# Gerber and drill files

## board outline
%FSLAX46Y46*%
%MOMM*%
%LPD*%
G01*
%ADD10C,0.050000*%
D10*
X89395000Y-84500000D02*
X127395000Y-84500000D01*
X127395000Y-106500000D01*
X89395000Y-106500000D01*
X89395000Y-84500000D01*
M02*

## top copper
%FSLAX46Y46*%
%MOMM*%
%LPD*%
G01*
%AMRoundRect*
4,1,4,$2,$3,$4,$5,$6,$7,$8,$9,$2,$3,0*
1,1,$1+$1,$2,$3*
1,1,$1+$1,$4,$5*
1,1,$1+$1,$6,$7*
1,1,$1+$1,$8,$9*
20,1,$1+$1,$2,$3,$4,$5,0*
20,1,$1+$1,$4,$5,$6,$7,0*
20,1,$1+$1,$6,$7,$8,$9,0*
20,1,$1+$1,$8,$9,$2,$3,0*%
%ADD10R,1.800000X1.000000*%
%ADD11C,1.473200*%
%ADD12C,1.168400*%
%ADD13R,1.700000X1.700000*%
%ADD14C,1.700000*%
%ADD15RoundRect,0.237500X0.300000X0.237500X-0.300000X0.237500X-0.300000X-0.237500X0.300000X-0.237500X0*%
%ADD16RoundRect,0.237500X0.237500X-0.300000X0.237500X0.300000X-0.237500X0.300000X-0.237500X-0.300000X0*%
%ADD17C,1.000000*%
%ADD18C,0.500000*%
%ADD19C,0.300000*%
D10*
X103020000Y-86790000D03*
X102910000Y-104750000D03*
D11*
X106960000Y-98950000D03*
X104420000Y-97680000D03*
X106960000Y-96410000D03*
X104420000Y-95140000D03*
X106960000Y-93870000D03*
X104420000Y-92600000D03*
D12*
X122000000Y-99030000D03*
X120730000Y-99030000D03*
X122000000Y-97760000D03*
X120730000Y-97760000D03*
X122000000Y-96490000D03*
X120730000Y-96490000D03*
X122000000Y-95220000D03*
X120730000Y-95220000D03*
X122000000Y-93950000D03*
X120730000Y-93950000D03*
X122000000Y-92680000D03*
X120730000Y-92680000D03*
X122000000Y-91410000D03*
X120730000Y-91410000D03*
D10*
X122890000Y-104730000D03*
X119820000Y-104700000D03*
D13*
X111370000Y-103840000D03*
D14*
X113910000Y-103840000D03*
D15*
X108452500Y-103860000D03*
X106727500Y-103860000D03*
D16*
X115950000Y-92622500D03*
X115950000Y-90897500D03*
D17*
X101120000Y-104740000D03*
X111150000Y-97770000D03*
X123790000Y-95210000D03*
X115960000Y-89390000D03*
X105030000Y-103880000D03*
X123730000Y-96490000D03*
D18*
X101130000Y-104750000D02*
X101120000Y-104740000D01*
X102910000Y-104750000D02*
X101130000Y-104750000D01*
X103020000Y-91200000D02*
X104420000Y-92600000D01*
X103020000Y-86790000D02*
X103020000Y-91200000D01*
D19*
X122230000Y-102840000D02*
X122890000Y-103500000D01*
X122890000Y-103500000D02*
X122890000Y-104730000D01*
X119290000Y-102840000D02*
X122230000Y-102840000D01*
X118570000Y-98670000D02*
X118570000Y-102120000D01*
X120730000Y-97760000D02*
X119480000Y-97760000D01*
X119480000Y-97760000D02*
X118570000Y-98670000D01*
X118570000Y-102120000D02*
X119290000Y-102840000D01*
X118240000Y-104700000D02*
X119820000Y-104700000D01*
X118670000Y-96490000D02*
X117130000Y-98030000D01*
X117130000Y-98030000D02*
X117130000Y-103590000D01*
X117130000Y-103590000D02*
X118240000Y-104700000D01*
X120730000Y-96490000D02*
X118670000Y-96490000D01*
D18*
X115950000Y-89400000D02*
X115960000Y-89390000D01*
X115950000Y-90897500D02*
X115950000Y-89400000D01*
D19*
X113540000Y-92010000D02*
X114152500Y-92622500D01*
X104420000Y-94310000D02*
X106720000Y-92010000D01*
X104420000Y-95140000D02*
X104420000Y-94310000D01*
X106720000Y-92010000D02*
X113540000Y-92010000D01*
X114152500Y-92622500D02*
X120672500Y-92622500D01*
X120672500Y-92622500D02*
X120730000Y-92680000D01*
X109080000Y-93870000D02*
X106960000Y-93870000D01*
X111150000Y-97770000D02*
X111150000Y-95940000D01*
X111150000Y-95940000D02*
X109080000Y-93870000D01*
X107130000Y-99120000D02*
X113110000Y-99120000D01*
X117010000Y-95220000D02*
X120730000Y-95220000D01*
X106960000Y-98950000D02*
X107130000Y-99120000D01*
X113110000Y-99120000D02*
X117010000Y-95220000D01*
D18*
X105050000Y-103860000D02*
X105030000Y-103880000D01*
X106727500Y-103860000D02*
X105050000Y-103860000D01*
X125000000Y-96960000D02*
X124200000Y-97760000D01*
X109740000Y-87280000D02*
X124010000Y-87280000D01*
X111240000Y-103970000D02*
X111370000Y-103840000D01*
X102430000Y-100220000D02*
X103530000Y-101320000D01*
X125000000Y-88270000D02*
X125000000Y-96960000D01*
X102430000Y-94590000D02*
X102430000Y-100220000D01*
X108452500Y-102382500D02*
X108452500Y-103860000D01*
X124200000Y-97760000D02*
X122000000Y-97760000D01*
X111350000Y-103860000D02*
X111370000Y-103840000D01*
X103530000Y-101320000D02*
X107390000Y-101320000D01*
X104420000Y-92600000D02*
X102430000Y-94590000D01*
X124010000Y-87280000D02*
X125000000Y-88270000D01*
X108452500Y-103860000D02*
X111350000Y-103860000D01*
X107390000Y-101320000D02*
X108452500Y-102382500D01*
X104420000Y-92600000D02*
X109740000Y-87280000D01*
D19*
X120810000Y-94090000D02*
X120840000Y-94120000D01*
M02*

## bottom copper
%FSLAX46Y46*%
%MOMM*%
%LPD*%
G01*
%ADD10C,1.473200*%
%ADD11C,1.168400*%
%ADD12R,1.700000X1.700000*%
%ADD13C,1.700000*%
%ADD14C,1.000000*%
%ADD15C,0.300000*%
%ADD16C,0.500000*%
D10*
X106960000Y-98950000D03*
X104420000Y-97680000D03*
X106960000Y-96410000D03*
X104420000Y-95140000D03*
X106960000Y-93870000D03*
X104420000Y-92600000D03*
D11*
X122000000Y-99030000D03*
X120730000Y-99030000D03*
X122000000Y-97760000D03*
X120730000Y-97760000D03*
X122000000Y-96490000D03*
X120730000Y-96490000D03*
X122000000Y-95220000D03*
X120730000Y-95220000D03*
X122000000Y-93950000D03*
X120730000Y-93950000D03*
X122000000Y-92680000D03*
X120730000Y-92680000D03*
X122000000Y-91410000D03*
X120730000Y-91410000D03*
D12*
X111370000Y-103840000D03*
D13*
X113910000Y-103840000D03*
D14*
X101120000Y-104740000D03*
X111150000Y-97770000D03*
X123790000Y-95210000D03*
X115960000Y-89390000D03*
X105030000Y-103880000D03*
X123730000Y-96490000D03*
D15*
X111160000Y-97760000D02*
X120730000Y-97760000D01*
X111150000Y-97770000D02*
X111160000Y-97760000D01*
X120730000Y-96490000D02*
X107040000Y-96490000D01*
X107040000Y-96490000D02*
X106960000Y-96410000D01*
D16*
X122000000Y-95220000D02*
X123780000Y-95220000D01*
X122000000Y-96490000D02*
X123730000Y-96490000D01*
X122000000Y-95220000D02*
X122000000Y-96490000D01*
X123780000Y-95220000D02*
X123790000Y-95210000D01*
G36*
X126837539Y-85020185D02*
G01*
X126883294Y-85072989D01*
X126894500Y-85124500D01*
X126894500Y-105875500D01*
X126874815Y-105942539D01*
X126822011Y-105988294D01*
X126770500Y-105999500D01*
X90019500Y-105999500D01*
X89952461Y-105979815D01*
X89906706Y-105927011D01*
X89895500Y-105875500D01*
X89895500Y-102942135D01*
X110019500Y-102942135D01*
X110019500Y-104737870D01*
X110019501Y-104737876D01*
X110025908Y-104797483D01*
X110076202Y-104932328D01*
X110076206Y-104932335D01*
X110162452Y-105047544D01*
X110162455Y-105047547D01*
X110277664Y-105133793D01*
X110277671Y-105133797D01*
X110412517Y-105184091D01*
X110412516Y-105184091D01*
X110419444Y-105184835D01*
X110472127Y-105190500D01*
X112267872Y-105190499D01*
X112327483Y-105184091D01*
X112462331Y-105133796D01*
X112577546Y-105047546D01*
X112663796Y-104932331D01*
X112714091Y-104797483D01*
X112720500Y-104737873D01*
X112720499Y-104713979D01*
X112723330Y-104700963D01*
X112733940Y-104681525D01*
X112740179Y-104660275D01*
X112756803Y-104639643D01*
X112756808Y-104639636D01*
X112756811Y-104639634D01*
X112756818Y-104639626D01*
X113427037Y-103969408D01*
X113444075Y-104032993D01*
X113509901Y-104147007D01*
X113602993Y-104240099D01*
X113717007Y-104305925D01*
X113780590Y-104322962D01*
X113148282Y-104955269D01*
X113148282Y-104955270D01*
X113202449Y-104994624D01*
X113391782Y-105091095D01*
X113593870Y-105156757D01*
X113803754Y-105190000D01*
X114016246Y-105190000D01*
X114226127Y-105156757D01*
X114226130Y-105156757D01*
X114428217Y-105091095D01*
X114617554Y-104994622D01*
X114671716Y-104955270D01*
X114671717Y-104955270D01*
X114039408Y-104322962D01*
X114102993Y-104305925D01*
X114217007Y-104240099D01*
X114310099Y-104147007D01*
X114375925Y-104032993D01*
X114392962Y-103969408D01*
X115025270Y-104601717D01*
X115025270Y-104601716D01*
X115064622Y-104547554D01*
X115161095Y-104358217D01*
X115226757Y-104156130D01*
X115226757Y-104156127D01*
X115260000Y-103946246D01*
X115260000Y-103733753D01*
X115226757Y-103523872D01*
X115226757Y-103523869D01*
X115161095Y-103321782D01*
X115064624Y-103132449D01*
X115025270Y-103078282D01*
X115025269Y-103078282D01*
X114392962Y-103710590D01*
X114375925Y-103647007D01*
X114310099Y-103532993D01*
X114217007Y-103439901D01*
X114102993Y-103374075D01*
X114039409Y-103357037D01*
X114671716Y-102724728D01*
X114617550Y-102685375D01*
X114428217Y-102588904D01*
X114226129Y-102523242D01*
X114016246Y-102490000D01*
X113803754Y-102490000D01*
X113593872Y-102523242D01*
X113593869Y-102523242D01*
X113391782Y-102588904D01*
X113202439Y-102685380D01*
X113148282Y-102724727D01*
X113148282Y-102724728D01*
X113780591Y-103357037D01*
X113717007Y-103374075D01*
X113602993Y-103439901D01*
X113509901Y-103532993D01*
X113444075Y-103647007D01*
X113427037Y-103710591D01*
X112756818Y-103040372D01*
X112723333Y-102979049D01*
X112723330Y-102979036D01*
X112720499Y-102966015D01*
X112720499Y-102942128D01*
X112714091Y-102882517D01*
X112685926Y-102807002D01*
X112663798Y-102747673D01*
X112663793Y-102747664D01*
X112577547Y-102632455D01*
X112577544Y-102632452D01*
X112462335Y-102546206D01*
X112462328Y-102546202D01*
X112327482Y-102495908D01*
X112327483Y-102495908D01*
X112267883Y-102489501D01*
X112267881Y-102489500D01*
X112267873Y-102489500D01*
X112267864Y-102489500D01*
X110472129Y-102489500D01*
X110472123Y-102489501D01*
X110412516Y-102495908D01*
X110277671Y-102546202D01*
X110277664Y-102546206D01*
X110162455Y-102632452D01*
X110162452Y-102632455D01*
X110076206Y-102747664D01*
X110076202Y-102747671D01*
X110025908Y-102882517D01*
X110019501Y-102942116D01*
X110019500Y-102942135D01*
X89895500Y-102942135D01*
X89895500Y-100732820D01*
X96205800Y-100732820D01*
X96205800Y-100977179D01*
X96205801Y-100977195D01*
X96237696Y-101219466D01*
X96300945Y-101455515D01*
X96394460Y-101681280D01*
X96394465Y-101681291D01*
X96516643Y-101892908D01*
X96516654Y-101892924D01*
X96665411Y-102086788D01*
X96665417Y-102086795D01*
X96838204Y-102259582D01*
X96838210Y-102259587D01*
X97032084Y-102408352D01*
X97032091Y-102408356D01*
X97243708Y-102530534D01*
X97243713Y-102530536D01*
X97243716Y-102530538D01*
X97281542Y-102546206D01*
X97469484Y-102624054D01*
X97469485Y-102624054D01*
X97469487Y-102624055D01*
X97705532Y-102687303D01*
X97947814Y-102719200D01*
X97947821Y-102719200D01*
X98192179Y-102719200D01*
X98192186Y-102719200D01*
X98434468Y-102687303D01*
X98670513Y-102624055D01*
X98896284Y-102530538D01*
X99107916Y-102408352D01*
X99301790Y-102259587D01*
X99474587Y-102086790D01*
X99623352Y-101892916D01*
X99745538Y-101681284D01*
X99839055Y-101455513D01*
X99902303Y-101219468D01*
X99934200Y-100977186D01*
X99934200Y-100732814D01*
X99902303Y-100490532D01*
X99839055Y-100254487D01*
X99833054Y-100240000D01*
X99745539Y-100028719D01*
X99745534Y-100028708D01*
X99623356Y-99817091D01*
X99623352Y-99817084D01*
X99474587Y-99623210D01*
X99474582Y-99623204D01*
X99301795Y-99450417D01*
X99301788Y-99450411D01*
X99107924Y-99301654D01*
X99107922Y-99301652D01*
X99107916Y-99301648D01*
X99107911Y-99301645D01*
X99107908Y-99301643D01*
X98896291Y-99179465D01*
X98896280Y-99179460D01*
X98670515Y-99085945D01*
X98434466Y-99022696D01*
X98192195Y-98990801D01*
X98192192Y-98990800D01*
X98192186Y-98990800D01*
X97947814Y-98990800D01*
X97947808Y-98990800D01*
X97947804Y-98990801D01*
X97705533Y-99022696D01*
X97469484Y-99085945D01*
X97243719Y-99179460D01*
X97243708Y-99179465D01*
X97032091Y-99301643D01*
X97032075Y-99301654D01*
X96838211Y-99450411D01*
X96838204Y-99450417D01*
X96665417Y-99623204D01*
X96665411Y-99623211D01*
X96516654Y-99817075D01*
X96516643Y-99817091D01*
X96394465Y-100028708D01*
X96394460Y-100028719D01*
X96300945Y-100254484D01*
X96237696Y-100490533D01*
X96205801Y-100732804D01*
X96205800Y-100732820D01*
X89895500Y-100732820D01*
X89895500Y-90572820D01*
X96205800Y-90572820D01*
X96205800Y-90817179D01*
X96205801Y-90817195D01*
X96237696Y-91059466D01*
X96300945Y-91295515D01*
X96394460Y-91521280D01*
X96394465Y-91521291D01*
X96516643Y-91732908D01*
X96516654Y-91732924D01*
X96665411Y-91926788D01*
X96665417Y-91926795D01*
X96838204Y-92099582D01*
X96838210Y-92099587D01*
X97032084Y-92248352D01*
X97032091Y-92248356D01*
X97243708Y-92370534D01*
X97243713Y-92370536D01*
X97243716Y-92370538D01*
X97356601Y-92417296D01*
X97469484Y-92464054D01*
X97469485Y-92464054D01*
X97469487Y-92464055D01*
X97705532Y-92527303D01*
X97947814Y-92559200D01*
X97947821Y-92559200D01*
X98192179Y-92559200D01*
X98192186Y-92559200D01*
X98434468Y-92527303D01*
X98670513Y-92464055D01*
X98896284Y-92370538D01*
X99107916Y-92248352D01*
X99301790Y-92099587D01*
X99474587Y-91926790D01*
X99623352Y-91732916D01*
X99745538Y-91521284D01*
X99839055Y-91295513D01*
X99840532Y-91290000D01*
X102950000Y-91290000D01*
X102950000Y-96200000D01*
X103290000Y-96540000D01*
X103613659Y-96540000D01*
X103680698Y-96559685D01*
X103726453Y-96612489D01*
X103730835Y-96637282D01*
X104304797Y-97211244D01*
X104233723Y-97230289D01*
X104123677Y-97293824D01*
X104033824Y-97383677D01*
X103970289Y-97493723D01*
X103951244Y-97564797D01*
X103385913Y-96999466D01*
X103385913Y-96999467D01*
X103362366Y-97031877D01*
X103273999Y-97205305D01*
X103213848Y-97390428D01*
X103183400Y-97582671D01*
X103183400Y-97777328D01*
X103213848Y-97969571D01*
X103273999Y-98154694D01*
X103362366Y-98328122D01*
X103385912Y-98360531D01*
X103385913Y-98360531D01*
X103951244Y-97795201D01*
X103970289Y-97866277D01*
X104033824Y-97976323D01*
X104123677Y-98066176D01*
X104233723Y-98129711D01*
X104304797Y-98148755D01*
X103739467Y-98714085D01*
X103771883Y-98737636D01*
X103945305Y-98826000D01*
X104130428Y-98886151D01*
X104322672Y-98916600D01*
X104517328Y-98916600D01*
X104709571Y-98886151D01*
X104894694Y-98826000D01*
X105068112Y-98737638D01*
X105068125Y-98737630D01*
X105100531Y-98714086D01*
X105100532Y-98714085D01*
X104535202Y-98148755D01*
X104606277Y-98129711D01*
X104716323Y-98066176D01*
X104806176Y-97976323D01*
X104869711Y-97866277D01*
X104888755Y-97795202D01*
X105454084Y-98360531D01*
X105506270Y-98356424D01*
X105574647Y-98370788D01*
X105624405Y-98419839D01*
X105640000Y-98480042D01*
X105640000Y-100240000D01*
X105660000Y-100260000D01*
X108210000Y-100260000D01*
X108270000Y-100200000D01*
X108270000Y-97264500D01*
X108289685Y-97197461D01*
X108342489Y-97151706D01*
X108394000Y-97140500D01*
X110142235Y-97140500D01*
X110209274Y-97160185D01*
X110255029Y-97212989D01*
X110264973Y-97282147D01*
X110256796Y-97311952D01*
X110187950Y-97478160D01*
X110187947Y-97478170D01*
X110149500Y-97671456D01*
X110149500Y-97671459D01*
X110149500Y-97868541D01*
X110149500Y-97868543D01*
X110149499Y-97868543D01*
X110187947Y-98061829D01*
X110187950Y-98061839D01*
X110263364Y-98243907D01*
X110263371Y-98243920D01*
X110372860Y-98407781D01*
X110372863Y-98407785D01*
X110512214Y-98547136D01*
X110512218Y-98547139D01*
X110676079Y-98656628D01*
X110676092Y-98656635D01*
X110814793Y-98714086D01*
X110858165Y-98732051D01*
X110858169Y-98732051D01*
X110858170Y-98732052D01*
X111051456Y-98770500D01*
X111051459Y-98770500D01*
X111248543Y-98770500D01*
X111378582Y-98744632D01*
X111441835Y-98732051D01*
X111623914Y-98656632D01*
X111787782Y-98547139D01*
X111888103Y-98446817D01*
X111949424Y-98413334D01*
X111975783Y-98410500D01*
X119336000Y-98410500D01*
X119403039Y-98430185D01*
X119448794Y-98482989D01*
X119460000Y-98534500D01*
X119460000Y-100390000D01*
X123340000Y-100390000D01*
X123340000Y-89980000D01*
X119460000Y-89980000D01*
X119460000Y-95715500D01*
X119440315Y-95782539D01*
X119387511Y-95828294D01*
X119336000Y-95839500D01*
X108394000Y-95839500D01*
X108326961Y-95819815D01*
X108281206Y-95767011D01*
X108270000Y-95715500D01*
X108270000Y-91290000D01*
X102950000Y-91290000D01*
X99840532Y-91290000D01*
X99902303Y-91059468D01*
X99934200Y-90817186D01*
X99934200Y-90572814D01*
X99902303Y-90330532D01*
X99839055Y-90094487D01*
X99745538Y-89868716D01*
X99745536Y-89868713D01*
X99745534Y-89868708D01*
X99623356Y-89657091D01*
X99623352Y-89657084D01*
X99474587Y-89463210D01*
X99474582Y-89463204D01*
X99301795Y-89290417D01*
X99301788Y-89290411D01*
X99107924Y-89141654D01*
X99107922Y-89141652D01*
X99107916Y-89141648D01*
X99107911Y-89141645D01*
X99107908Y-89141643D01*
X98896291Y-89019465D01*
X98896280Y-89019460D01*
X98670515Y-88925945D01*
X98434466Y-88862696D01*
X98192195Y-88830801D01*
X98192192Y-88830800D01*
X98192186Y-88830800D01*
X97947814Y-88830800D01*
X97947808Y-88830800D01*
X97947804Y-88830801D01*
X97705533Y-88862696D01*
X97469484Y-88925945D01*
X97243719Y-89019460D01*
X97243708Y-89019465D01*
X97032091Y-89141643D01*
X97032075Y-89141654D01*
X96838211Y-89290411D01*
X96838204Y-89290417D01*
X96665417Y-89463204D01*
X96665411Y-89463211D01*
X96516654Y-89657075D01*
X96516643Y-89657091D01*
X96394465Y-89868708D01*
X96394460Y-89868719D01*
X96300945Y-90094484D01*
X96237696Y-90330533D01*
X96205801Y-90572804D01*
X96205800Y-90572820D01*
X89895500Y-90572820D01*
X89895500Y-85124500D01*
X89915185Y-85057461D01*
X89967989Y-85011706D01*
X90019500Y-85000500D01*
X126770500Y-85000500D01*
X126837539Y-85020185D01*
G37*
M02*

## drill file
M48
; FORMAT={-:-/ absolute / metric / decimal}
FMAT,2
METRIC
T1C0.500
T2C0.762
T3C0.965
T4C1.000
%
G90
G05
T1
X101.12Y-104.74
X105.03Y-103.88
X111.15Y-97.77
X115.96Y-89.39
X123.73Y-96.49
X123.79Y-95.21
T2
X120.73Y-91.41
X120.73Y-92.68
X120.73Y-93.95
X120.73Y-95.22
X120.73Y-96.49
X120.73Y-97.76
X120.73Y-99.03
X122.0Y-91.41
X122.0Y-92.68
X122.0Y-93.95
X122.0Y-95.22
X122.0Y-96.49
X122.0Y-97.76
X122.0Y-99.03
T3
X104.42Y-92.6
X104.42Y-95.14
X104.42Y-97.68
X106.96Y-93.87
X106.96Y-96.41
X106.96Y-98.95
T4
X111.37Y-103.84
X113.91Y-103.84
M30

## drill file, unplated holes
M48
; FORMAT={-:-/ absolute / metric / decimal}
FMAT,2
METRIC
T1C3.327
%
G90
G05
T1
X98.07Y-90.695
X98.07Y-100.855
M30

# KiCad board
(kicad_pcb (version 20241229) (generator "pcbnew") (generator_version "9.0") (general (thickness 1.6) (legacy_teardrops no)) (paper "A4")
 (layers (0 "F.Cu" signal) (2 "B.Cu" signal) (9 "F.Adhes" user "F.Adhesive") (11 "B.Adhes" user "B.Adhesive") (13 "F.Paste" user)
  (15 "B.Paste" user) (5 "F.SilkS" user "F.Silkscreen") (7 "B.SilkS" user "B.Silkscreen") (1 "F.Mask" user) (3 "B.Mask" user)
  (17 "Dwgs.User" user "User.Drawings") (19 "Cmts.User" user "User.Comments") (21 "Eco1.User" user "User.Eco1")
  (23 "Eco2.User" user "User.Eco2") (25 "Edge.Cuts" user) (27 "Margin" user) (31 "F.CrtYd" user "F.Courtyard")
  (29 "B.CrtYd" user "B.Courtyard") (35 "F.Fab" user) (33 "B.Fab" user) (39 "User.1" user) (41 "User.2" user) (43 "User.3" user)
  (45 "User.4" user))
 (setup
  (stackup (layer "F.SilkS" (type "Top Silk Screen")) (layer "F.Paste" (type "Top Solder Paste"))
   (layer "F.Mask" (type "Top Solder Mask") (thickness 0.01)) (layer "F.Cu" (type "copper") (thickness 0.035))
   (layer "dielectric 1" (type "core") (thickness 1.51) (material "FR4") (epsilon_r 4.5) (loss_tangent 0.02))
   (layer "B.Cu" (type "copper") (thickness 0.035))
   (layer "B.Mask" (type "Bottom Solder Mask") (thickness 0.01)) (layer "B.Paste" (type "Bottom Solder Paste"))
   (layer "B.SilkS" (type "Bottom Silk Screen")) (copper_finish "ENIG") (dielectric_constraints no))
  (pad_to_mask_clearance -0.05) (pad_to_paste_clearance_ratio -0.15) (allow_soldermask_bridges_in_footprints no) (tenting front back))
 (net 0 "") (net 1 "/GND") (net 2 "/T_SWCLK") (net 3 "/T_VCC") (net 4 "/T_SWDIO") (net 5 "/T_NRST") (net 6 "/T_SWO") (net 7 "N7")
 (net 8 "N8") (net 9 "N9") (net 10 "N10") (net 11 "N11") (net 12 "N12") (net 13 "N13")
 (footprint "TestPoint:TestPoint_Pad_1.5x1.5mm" (layer "F.Cu") (at 102.91 104.75)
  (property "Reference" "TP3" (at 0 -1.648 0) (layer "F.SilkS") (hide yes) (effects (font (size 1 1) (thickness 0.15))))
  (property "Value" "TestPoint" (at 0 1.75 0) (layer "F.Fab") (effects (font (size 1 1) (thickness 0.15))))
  (pad "1" smd rect (at 0 0) (size 1.8 1) (layers "F.Cu" "F.Mask") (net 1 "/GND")))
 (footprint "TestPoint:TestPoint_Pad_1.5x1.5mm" (layer "F.Cu") (at 119.82 104.7 180)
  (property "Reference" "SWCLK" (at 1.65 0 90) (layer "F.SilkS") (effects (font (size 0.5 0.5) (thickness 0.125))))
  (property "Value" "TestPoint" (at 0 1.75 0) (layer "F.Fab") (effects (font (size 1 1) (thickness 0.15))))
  (pad "1" smd rect (at 0 0 180) (size 1.8 1) (layers "F.Cu" "F.Mask") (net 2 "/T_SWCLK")))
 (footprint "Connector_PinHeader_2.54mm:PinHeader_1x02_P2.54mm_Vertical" (layer "F.Cu") (at 111.37 103.84 90)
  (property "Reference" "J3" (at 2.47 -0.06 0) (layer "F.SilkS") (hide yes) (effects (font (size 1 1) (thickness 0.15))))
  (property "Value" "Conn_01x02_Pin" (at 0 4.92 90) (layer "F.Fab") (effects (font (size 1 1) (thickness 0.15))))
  (pad "1" thru_hole rect (at 0 0 90) (size 1.7 1.7) (drill 1) (layers "*.Cu" "*.Mask") (remove_unused_layers no) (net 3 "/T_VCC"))
  (pad "2" thru_hole circle (at 0 2.54 90) (size 1.7 1.7) (drill 1) (layers "*.Cu" "*.Mask") (remove_unused_layers no) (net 1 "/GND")))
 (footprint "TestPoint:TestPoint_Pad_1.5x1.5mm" (layer "F.Cu") (at 103.02 86.79)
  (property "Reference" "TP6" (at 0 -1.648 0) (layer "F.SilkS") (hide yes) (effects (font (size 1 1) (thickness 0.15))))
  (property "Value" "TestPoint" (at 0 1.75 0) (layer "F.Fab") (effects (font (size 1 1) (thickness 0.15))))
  (pad "1" smd rect (at 0 0) (size 1.8 1) (layers "F.Cu" "F.Mask") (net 3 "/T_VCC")))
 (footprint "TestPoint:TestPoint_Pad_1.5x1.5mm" (layer "F.Cu") (at 122.89 104.73 180)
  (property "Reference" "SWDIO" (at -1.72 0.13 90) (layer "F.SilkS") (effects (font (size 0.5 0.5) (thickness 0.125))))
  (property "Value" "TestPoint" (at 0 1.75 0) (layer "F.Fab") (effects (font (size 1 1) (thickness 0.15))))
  (pad "1" smd rect (at 0 0 180) (size 1.8 1) (layers "F.Cu" "F.Mask") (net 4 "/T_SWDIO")))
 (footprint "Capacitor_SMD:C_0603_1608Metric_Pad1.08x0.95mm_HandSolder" (layer "F.Cu") (at 107.59 103.86 180)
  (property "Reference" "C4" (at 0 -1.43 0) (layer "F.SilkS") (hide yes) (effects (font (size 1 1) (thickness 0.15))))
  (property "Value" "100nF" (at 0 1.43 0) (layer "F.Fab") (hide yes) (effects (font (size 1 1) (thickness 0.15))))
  (pad "1" smd roundrect (at -0.8625 0 180) (size 1.075 0.95) (layers "F.Cu" "F.Mask" "F.Paste") (roundrect_rratio 0.25) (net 3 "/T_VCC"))
  (pad "2" smd roundrect (at 0.8625 0 180) (size 1.075 0.95) (layers "F.Cu" "F.Mask" "F.Paste") (roundrect_rratio 0.25) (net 1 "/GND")))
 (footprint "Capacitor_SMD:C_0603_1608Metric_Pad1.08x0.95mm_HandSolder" (layer "F.Cu") (at 115.95 91.76 90)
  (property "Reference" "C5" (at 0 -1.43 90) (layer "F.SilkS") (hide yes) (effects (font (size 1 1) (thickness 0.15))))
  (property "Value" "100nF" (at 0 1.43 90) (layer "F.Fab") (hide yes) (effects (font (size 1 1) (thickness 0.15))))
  (pad "1" smd roundrect (at -0.8625 0 90) (size 1.075 0.95) (layers "F.Cu" "F.Mask" "F.Paste") (roundrect_rratio 0.25) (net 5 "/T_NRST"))
  (pad "2" smd roundrect (at 0.8625 0 90) (size 1.075 0.95) (layers "F.Cu" "F.Mask" "F.Paste") (roundrect_rratio 0.25) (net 1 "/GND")))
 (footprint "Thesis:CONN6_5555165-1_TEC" (layer "B.Cu") (at 106.96 98.95 90)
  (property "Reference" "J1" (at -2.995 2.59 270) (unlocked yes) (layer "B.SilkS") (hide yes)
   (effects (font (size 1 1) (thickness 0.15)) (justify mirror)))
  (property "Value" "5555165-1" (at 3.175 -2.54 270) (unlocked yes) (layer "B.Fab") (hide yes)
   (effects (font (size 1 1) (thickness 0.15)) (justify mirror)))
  (pad "" np_thru_hole circle (at -1.905 -8.89 90) (size 3.3274 3.3274) (drill 3.3274) (layers "*.Cu" "*.Mask"))
  (pad "" np_thru_hole circle (at 8.255 -8.89 90) (size 3.3274 3.3274) (drill 3.3274) (layers "*.Cu" "*.Mask"))
  (pad "1" thru_hole circle (at 0 0 90) (size 1.4732 1.4732) (drill 0.9652) (layers "*.Cu" "*.Mask") (remove_unused_layers no)
   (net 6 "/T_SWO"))
  (pad "2" thru_hole circle (at 1.27 -2.54 90) (size 1.4732 1.4732) (drill 0.9652) (layers "*.Cu" "*.Mask") (remove_unused_layers no)
   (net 1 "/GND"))
  (pad "3" thru_hole circle (at 2.54 0 90) (size 1.4732 1.4732) (drill 0.9652) (layers "*.Cu" "*.Mask") (remove_unused_layers no)
   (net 2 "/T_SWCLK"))
  (pad "4" thru_hole circle (at 3.81 -2.54 90) (size 1.4732 1.4732) (drill 0.9652) (layers "*.Cu" "*.Mask") (remove_unused_layers no)
   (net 5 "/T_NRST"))
  (pad "5" thru_hole circle (at 5.08 0 90) (size 1.4732 1.4732) (drill 0.9652) (layers "*.Cu" "*.Mask") (remove_unused_layers no)
   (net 4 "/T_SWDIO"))
  (pad "6" thru_hole circle (at 6.35 -2.54 90) (size 1.4732 1.4732) (drill 0.9652) (layers "*.Cu" "*.Mask") (remove_unused_layers no)
   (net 3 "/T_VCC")))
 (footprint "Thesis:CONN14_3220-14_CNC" (layer "B.Cu") (at 122 99.03 90)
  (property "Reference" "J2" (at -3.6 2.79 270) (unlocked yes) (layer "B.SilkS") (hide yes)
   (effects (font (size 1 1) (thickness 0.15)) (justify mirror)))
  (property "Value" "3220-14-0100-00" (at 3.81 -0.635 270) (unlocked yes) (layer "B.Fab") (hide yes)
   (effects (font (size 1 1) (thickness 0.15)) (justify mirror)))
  (pad "1" thru_hole circle (at 0 0 90) (size 1.1684 1.1684) (drill 0.762) (layers "*.Cu" "*.Mask") (remove_unused_layers no) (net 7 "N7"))
  (pad "2" thru_hole circle (at 0 -1.27 90) (size 1.1684 1.1684) (drill 0.762) (layers "*.Cu" "*.Mask") (remove_unused_layers no)
   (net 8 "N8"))
  (pad "3" thru_hole circle (at 1.27 0 90) (size 1.1684 1.1684) (drill 0.762) (layers "*.Cu" "*.Mask") (remove_unused_layers no)
   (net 3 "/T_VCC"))
  (pad "4" thru_hole circle (at 1.27 -1.27 90) (size 1.1684 1.1684) (drill 0.762) (layers "*.Cu" "*.Mask") (remove_unused_layers no)
   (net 4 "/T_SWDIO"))
  (pad "5" thru_hole circle (at 2.54 0 90) (size 1.1684 1.1684) (drill 0.762) (layers "*.Cu" "*.Mask") (remove_unused_layers no)
   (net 1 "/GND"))
  (pad "6" thru_hole circle (at 2.54 -1.27 90) (size 1.1684 1.1684) (drill 0.762) (layers "*.Cu" "*.Mask") (remove_unused_layers no)
   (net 2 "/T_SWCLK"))
  (pad "7" thru_hole circle (at 3.81 0 90) (size 1.1684 1.1684) (drill 0.762) (layers "*.Cu" "*.Mask") (remove_unused_layers no)
   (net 1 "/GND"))
  (pad "8" thru_hole circle (at 3.81 -1.27 90) (size 1.1684 1.1684) (drill 0.762) (layers "*.Cu" "*.Mask") (remove_unused_layers no)
   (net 6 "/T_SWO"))
  (pad "9" thru_hole circle (at 5.08 0 90) (size 1.1684 1.1684) (drill 0.762) (layers "*.Cu" "*.Mask") (remove_unused_layers no)
   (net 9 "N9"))
  (pad "10" thru_hole circle (at 5.08 -1.27 90) (size 1.1684 1.1684) (drill 0.762) (layers "*.Cu" "*.Mask") (remove_unused_layers no)
   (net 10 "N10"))
  (pad "11" thru_hole circle (at 6.35 0 90) (size 1.1684 1.1684) (drill 0.762) (layers "*.Cu" "*.Mask") (remove_unused_layers no)
   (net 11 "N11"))
  (pad "12" thru_hole circle (at 6.35 -1.27 90) (size 1.1684 1.1684) (drill 0.762) (layers "*.Cu" "*.Mask") (remove_unused_layers no)
   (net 5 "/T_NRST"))
  (pad "13" thru_hole circle (at 7.62 0 90) (size 1.1684 1.1684) (drill 0.762) (layers "*.Cu" "*.Mask") (remove_unused_layers no)
   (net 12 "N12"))
  (pad "14" thru_hole circle (at 7.62 -1.27 90) (size 1.1684 1.1684) (drill 0.762) (layers "*.Cu" "*.Mask") (remove_unused_layers no)
   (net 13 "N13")))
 (gr_rect (start 89.395 84.5) (end 127.395 106.5) (stroke (width 0.05) (type solid)) (fill no) (layer "Edge.Cuts"))
 (segment (start 122.23 102.84) (end 122.89 103.5) (width 0.3) (layer "F.Cu") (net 4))
 (segment (start 109.08 93.87) (end 106.96 93.87) (width 0.3) (layer "F.Cu") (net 4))
 (segment (start 118.57 98.67) (end 118.57 102.12) (width 0.3) (layer "F.Cu") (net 4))
 (segment (start 122.89 103.5) (end 122.89 104.73) (width 0.3) (layer "F.Cu") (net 4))
 (segment (start 118.57 102.12) (end 119.29 102.84) (width 0.3) (layer "F.Cu") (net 4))
 (segment (start 111.15 97.77) (end 111.15 95.94) (width 0.3) (layer "F.Cu") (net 4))
 (segment (start 119.48 97.76) (end 118.57 98.67) (width 0.3) (layer "F.Cu") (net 4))
 (segment (start 111.15 95.94) (end 109.08 93.87) (width 0.3) (layer "F.Cu") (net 4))
 (segment (start 120.73 97.76) (end 119.48 97.76) (width 0.3) (layer "F.Cu") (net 4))
 (segment (start 119.29 102.84) (end 122.23 102.84) (width 0.3) (layer "F.Cu") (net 4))
 (via (at 111.15 97.77) (size 1) (drill 0.5) (layers "F.Cu" "B.Cu") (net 4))
 (segment (start 111.16 97.76) (end 120.73 97.76) (width 0.3) (layer "B.Cu") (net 4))
 (segment (start 111.15 97.77) (end 111.16 97.76) (width 0.3) (layer "B.Cu") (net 4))
 (segment (start 104.42 94.31) (end 106.72 92.01) (width 0.3) (layer "F.Cu") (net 5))
 (segment (start 114.1525 92.6225) (end 120.6725 92.6225) (width 0.3) (layer "F.Cu") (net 5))
 (segment (start 106.72 92.01) (end 113.54 92.01) (width 0.3) (layer "F.Cu") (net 5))
 (segment (start 113.54 92.01) (end 114.1525 92.6225) (width 0.3) (layer "F.Cu") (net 5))
 (segment (start 104.42 95.14) (end 104.42 94.31) (width 0.3) (layer "F.Cu") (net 5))
 (segment (start 120.6725 92.6225) (end 120.73 92.68) (width 0.3) (layer "F.Cu") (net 5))
 (segment (start 117.13 98.03) (end 117.13 103.59) (width 0.3) (layer "F.Cu") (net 2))
 (segment (start 118.67 96.49) (end 117.13 98.03) (width 0.3) (layer "F.Cu") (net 2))
 (segment (start 117.13 103.59) (end 118.24 104.7) (width 0.3) (layer "F.Cu") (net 2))
 (segment (start 120.73 96.49) (end 118.67 96.49) (width 0.3) (layer "F.Cu") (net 2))
 (segment (start 118.24 104.7) (end 119.82 104.7) (width 0.3) (layer "F.Cu") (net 2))
 (segment (start 120.73 96.49) (end 107.04 96.49) (width 0.3) (layer "B.Cu") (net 2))
 (segment (start 107.04 96.49) (end 106.96 96.41) (width 0.3) (layer "B.Cu") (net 2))
 (segment (start 107.13 99.12) (end 113.11 99.12) (width 0.3) (layer "F.Cu") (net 6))
 (segment (start 117.01 95.22) (end 120.73 95.22) (width 0.3) (layer "F.Cu") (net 6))
 (segment (start 106.96 98.95) (end 107.13 99.12) (width 0.3) (layer "F.Cu") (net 6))
 (segment (start 113.11 99.12) (end 117.01 95.22) (width 0.3) (layer "F.Cu") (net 6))
 (segment (start 102.91 104.75) (end 101.13 104.75) (width 0.5) (layer "F.Cu") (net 1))
 (segment (start 105.05 103.86) (end 105.03 103.88) (width 0.5) (layer "F.Cu") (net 1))
 (segment (start 115.95 90.8975) (end 115.95 89.4) (width 0.5) (layer "F.Cu") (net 1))
 (segment (start 115.95 89.4) (end 115.96 89.39) (width 0.5) (layer "F.Cu") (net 1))
 (segment (start 106.7275 103.86) (end 105.05 103.86) (width 0.5) (layer "F.Cu") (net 1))
 (segment (start 101.13 104.75) (end 101.12 104.74) (width 0.5) (layer "F.Cu") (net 1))
 (via (at 123.79 95.21) (size 1) (drill 0.5) (layers "F.Cu" "B.Cu") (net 1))
 (via (at 115.96 89.39) (size 1) (drill 0.5) (layers "F.Cu" "B.Cu") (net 1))
 (via (at 105.03 103.88) (size 1) (drill 0.5) (layers "F.Cu" "B.Cu") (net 1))
 (via (at 123.73 96.49) (size 1) (drill 0.5) (layers "F.Cu" "B.Cu") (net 1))
 (via (at 101.12 104.74) (size 1) (drill 0.5) (layers "F.Cu" "B.Cu") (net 1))
 (segment (start 122 95.22) (end 123.78 95.22) (width 0.5) (layer "B.Cu") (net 1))
 (segment (start 122 96.49) (end 123.73 96.49) (width 0.5) (layer "B.Cu") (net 1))
 (segment (start 122 95.22) (end 122 96.49) (width 0.5) (layer "B.Cu") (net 1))
 (segment (start 123.78 95.22) (end 123.79 95.21) (width 0.5) (layer "B.Cu") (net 1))
 (segment (start 125 96.96) (end 124.2 97.76) (width 0.5) (layer "F.Cu") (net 3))
 (segment (start 109.74 87.28) (end 124.01 87.28) (width 0.5) (layer "F.Cu") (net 3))
 (segment (start 111.24 103.97) (end 111.37 103.84) (width 0.5) (layer "F.Cu") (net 3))
 (segment (start 102.43 100.22) (end 103.53 101.32) (width 0.5) (layer "F.Cu") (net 3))
 (segment (start 125 88.27) (end 125 96.96) (width 0.5) (layer "F.Cu") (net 3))
 (segment (start 103.02 91.2) (end 104.42 92.6) (width 0.5) (layer "F.Cu") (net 3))
 (segment (start 102.43 94.59) (end 102.43 100.22) (width 0.5) (layer "F.Cu") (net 3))
 (segment (start 103.02 86.79) (end 103.02 91.2) (width 0.5) (layer "F.Cu") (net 3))
 (segment (start 108.4525 102.3825) (end 108.4525 103.86) (width 0.5) (layer "F.Cu") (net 3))
 (segment (start 124.2 97.76) (end 122 97.76) (width 0.5) (layer "F.Cu") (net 3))
 (segment (start 111.35 103.86) (end 111.37 103.84) (width 0.5) (layer "F.Cu") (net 3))
 (segment (start 103.53 101.32) (end 107.39 101.32) (width 0.5) (layer "F.Cu") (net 3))
 (segment (start 104.42 92.6) (end 102.43 94.59) (width 0.5) (layer "F.Cu") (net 3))
 (segment (start 124.01 87.28) (end 125 88.27) (width 0.5) (layer "F.Cu") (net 3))
 (segment (start 108.4525 103.86) (end 111.35 103.86) (width 0.5) (layer "F.Cu") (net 3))
 (segment (start 107.39 101.32) (end 108.4525 102.3825) (width 0.5) (layer "F.Cu") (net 3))
 (segment (start 104.42 92.6) (end 109.74 87.28) (width 0.5) (layer "F.Cu") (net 3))
 (segment (start 120.81 94.09) (end 120.84 94.12) (width 0.3) (layer "F.Cu") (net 10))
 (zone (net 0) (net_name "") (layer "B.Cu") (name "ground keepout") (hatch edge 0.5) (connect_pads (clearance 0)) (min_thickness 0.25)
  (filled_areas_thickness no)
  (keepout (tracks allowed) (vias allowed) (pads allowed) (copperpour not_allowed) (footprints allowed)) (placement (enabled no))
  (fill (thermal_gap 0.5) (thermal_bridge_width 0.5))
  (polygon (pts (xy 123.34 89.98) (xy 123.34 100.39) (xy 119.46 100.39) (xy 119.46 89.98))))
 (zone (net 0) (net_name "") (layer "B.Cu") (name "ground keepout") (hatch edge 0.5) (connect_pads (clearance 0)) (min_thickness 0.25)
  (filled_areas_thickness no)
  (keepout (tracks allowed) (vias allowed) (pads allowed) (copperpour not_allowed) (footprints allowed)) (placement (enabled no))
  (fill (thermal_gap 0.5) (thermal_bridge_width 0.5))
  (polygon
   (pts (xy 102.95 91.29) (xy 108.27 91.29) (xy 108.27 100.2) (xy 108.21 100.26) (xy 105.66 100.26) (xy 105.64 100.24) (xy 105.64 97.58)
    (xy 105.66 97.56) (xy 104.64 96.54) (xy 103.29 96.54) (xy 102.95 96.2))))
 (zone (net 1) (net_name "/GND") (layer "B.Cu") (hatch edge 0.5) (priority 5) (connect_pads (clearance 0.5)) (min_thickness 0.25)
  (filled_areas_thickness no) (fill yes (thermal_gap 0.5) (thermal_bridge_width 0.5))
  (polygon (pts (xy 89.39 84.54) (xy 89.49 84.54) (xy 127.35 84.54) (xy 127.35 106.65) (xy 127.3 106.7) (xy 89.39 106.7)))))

